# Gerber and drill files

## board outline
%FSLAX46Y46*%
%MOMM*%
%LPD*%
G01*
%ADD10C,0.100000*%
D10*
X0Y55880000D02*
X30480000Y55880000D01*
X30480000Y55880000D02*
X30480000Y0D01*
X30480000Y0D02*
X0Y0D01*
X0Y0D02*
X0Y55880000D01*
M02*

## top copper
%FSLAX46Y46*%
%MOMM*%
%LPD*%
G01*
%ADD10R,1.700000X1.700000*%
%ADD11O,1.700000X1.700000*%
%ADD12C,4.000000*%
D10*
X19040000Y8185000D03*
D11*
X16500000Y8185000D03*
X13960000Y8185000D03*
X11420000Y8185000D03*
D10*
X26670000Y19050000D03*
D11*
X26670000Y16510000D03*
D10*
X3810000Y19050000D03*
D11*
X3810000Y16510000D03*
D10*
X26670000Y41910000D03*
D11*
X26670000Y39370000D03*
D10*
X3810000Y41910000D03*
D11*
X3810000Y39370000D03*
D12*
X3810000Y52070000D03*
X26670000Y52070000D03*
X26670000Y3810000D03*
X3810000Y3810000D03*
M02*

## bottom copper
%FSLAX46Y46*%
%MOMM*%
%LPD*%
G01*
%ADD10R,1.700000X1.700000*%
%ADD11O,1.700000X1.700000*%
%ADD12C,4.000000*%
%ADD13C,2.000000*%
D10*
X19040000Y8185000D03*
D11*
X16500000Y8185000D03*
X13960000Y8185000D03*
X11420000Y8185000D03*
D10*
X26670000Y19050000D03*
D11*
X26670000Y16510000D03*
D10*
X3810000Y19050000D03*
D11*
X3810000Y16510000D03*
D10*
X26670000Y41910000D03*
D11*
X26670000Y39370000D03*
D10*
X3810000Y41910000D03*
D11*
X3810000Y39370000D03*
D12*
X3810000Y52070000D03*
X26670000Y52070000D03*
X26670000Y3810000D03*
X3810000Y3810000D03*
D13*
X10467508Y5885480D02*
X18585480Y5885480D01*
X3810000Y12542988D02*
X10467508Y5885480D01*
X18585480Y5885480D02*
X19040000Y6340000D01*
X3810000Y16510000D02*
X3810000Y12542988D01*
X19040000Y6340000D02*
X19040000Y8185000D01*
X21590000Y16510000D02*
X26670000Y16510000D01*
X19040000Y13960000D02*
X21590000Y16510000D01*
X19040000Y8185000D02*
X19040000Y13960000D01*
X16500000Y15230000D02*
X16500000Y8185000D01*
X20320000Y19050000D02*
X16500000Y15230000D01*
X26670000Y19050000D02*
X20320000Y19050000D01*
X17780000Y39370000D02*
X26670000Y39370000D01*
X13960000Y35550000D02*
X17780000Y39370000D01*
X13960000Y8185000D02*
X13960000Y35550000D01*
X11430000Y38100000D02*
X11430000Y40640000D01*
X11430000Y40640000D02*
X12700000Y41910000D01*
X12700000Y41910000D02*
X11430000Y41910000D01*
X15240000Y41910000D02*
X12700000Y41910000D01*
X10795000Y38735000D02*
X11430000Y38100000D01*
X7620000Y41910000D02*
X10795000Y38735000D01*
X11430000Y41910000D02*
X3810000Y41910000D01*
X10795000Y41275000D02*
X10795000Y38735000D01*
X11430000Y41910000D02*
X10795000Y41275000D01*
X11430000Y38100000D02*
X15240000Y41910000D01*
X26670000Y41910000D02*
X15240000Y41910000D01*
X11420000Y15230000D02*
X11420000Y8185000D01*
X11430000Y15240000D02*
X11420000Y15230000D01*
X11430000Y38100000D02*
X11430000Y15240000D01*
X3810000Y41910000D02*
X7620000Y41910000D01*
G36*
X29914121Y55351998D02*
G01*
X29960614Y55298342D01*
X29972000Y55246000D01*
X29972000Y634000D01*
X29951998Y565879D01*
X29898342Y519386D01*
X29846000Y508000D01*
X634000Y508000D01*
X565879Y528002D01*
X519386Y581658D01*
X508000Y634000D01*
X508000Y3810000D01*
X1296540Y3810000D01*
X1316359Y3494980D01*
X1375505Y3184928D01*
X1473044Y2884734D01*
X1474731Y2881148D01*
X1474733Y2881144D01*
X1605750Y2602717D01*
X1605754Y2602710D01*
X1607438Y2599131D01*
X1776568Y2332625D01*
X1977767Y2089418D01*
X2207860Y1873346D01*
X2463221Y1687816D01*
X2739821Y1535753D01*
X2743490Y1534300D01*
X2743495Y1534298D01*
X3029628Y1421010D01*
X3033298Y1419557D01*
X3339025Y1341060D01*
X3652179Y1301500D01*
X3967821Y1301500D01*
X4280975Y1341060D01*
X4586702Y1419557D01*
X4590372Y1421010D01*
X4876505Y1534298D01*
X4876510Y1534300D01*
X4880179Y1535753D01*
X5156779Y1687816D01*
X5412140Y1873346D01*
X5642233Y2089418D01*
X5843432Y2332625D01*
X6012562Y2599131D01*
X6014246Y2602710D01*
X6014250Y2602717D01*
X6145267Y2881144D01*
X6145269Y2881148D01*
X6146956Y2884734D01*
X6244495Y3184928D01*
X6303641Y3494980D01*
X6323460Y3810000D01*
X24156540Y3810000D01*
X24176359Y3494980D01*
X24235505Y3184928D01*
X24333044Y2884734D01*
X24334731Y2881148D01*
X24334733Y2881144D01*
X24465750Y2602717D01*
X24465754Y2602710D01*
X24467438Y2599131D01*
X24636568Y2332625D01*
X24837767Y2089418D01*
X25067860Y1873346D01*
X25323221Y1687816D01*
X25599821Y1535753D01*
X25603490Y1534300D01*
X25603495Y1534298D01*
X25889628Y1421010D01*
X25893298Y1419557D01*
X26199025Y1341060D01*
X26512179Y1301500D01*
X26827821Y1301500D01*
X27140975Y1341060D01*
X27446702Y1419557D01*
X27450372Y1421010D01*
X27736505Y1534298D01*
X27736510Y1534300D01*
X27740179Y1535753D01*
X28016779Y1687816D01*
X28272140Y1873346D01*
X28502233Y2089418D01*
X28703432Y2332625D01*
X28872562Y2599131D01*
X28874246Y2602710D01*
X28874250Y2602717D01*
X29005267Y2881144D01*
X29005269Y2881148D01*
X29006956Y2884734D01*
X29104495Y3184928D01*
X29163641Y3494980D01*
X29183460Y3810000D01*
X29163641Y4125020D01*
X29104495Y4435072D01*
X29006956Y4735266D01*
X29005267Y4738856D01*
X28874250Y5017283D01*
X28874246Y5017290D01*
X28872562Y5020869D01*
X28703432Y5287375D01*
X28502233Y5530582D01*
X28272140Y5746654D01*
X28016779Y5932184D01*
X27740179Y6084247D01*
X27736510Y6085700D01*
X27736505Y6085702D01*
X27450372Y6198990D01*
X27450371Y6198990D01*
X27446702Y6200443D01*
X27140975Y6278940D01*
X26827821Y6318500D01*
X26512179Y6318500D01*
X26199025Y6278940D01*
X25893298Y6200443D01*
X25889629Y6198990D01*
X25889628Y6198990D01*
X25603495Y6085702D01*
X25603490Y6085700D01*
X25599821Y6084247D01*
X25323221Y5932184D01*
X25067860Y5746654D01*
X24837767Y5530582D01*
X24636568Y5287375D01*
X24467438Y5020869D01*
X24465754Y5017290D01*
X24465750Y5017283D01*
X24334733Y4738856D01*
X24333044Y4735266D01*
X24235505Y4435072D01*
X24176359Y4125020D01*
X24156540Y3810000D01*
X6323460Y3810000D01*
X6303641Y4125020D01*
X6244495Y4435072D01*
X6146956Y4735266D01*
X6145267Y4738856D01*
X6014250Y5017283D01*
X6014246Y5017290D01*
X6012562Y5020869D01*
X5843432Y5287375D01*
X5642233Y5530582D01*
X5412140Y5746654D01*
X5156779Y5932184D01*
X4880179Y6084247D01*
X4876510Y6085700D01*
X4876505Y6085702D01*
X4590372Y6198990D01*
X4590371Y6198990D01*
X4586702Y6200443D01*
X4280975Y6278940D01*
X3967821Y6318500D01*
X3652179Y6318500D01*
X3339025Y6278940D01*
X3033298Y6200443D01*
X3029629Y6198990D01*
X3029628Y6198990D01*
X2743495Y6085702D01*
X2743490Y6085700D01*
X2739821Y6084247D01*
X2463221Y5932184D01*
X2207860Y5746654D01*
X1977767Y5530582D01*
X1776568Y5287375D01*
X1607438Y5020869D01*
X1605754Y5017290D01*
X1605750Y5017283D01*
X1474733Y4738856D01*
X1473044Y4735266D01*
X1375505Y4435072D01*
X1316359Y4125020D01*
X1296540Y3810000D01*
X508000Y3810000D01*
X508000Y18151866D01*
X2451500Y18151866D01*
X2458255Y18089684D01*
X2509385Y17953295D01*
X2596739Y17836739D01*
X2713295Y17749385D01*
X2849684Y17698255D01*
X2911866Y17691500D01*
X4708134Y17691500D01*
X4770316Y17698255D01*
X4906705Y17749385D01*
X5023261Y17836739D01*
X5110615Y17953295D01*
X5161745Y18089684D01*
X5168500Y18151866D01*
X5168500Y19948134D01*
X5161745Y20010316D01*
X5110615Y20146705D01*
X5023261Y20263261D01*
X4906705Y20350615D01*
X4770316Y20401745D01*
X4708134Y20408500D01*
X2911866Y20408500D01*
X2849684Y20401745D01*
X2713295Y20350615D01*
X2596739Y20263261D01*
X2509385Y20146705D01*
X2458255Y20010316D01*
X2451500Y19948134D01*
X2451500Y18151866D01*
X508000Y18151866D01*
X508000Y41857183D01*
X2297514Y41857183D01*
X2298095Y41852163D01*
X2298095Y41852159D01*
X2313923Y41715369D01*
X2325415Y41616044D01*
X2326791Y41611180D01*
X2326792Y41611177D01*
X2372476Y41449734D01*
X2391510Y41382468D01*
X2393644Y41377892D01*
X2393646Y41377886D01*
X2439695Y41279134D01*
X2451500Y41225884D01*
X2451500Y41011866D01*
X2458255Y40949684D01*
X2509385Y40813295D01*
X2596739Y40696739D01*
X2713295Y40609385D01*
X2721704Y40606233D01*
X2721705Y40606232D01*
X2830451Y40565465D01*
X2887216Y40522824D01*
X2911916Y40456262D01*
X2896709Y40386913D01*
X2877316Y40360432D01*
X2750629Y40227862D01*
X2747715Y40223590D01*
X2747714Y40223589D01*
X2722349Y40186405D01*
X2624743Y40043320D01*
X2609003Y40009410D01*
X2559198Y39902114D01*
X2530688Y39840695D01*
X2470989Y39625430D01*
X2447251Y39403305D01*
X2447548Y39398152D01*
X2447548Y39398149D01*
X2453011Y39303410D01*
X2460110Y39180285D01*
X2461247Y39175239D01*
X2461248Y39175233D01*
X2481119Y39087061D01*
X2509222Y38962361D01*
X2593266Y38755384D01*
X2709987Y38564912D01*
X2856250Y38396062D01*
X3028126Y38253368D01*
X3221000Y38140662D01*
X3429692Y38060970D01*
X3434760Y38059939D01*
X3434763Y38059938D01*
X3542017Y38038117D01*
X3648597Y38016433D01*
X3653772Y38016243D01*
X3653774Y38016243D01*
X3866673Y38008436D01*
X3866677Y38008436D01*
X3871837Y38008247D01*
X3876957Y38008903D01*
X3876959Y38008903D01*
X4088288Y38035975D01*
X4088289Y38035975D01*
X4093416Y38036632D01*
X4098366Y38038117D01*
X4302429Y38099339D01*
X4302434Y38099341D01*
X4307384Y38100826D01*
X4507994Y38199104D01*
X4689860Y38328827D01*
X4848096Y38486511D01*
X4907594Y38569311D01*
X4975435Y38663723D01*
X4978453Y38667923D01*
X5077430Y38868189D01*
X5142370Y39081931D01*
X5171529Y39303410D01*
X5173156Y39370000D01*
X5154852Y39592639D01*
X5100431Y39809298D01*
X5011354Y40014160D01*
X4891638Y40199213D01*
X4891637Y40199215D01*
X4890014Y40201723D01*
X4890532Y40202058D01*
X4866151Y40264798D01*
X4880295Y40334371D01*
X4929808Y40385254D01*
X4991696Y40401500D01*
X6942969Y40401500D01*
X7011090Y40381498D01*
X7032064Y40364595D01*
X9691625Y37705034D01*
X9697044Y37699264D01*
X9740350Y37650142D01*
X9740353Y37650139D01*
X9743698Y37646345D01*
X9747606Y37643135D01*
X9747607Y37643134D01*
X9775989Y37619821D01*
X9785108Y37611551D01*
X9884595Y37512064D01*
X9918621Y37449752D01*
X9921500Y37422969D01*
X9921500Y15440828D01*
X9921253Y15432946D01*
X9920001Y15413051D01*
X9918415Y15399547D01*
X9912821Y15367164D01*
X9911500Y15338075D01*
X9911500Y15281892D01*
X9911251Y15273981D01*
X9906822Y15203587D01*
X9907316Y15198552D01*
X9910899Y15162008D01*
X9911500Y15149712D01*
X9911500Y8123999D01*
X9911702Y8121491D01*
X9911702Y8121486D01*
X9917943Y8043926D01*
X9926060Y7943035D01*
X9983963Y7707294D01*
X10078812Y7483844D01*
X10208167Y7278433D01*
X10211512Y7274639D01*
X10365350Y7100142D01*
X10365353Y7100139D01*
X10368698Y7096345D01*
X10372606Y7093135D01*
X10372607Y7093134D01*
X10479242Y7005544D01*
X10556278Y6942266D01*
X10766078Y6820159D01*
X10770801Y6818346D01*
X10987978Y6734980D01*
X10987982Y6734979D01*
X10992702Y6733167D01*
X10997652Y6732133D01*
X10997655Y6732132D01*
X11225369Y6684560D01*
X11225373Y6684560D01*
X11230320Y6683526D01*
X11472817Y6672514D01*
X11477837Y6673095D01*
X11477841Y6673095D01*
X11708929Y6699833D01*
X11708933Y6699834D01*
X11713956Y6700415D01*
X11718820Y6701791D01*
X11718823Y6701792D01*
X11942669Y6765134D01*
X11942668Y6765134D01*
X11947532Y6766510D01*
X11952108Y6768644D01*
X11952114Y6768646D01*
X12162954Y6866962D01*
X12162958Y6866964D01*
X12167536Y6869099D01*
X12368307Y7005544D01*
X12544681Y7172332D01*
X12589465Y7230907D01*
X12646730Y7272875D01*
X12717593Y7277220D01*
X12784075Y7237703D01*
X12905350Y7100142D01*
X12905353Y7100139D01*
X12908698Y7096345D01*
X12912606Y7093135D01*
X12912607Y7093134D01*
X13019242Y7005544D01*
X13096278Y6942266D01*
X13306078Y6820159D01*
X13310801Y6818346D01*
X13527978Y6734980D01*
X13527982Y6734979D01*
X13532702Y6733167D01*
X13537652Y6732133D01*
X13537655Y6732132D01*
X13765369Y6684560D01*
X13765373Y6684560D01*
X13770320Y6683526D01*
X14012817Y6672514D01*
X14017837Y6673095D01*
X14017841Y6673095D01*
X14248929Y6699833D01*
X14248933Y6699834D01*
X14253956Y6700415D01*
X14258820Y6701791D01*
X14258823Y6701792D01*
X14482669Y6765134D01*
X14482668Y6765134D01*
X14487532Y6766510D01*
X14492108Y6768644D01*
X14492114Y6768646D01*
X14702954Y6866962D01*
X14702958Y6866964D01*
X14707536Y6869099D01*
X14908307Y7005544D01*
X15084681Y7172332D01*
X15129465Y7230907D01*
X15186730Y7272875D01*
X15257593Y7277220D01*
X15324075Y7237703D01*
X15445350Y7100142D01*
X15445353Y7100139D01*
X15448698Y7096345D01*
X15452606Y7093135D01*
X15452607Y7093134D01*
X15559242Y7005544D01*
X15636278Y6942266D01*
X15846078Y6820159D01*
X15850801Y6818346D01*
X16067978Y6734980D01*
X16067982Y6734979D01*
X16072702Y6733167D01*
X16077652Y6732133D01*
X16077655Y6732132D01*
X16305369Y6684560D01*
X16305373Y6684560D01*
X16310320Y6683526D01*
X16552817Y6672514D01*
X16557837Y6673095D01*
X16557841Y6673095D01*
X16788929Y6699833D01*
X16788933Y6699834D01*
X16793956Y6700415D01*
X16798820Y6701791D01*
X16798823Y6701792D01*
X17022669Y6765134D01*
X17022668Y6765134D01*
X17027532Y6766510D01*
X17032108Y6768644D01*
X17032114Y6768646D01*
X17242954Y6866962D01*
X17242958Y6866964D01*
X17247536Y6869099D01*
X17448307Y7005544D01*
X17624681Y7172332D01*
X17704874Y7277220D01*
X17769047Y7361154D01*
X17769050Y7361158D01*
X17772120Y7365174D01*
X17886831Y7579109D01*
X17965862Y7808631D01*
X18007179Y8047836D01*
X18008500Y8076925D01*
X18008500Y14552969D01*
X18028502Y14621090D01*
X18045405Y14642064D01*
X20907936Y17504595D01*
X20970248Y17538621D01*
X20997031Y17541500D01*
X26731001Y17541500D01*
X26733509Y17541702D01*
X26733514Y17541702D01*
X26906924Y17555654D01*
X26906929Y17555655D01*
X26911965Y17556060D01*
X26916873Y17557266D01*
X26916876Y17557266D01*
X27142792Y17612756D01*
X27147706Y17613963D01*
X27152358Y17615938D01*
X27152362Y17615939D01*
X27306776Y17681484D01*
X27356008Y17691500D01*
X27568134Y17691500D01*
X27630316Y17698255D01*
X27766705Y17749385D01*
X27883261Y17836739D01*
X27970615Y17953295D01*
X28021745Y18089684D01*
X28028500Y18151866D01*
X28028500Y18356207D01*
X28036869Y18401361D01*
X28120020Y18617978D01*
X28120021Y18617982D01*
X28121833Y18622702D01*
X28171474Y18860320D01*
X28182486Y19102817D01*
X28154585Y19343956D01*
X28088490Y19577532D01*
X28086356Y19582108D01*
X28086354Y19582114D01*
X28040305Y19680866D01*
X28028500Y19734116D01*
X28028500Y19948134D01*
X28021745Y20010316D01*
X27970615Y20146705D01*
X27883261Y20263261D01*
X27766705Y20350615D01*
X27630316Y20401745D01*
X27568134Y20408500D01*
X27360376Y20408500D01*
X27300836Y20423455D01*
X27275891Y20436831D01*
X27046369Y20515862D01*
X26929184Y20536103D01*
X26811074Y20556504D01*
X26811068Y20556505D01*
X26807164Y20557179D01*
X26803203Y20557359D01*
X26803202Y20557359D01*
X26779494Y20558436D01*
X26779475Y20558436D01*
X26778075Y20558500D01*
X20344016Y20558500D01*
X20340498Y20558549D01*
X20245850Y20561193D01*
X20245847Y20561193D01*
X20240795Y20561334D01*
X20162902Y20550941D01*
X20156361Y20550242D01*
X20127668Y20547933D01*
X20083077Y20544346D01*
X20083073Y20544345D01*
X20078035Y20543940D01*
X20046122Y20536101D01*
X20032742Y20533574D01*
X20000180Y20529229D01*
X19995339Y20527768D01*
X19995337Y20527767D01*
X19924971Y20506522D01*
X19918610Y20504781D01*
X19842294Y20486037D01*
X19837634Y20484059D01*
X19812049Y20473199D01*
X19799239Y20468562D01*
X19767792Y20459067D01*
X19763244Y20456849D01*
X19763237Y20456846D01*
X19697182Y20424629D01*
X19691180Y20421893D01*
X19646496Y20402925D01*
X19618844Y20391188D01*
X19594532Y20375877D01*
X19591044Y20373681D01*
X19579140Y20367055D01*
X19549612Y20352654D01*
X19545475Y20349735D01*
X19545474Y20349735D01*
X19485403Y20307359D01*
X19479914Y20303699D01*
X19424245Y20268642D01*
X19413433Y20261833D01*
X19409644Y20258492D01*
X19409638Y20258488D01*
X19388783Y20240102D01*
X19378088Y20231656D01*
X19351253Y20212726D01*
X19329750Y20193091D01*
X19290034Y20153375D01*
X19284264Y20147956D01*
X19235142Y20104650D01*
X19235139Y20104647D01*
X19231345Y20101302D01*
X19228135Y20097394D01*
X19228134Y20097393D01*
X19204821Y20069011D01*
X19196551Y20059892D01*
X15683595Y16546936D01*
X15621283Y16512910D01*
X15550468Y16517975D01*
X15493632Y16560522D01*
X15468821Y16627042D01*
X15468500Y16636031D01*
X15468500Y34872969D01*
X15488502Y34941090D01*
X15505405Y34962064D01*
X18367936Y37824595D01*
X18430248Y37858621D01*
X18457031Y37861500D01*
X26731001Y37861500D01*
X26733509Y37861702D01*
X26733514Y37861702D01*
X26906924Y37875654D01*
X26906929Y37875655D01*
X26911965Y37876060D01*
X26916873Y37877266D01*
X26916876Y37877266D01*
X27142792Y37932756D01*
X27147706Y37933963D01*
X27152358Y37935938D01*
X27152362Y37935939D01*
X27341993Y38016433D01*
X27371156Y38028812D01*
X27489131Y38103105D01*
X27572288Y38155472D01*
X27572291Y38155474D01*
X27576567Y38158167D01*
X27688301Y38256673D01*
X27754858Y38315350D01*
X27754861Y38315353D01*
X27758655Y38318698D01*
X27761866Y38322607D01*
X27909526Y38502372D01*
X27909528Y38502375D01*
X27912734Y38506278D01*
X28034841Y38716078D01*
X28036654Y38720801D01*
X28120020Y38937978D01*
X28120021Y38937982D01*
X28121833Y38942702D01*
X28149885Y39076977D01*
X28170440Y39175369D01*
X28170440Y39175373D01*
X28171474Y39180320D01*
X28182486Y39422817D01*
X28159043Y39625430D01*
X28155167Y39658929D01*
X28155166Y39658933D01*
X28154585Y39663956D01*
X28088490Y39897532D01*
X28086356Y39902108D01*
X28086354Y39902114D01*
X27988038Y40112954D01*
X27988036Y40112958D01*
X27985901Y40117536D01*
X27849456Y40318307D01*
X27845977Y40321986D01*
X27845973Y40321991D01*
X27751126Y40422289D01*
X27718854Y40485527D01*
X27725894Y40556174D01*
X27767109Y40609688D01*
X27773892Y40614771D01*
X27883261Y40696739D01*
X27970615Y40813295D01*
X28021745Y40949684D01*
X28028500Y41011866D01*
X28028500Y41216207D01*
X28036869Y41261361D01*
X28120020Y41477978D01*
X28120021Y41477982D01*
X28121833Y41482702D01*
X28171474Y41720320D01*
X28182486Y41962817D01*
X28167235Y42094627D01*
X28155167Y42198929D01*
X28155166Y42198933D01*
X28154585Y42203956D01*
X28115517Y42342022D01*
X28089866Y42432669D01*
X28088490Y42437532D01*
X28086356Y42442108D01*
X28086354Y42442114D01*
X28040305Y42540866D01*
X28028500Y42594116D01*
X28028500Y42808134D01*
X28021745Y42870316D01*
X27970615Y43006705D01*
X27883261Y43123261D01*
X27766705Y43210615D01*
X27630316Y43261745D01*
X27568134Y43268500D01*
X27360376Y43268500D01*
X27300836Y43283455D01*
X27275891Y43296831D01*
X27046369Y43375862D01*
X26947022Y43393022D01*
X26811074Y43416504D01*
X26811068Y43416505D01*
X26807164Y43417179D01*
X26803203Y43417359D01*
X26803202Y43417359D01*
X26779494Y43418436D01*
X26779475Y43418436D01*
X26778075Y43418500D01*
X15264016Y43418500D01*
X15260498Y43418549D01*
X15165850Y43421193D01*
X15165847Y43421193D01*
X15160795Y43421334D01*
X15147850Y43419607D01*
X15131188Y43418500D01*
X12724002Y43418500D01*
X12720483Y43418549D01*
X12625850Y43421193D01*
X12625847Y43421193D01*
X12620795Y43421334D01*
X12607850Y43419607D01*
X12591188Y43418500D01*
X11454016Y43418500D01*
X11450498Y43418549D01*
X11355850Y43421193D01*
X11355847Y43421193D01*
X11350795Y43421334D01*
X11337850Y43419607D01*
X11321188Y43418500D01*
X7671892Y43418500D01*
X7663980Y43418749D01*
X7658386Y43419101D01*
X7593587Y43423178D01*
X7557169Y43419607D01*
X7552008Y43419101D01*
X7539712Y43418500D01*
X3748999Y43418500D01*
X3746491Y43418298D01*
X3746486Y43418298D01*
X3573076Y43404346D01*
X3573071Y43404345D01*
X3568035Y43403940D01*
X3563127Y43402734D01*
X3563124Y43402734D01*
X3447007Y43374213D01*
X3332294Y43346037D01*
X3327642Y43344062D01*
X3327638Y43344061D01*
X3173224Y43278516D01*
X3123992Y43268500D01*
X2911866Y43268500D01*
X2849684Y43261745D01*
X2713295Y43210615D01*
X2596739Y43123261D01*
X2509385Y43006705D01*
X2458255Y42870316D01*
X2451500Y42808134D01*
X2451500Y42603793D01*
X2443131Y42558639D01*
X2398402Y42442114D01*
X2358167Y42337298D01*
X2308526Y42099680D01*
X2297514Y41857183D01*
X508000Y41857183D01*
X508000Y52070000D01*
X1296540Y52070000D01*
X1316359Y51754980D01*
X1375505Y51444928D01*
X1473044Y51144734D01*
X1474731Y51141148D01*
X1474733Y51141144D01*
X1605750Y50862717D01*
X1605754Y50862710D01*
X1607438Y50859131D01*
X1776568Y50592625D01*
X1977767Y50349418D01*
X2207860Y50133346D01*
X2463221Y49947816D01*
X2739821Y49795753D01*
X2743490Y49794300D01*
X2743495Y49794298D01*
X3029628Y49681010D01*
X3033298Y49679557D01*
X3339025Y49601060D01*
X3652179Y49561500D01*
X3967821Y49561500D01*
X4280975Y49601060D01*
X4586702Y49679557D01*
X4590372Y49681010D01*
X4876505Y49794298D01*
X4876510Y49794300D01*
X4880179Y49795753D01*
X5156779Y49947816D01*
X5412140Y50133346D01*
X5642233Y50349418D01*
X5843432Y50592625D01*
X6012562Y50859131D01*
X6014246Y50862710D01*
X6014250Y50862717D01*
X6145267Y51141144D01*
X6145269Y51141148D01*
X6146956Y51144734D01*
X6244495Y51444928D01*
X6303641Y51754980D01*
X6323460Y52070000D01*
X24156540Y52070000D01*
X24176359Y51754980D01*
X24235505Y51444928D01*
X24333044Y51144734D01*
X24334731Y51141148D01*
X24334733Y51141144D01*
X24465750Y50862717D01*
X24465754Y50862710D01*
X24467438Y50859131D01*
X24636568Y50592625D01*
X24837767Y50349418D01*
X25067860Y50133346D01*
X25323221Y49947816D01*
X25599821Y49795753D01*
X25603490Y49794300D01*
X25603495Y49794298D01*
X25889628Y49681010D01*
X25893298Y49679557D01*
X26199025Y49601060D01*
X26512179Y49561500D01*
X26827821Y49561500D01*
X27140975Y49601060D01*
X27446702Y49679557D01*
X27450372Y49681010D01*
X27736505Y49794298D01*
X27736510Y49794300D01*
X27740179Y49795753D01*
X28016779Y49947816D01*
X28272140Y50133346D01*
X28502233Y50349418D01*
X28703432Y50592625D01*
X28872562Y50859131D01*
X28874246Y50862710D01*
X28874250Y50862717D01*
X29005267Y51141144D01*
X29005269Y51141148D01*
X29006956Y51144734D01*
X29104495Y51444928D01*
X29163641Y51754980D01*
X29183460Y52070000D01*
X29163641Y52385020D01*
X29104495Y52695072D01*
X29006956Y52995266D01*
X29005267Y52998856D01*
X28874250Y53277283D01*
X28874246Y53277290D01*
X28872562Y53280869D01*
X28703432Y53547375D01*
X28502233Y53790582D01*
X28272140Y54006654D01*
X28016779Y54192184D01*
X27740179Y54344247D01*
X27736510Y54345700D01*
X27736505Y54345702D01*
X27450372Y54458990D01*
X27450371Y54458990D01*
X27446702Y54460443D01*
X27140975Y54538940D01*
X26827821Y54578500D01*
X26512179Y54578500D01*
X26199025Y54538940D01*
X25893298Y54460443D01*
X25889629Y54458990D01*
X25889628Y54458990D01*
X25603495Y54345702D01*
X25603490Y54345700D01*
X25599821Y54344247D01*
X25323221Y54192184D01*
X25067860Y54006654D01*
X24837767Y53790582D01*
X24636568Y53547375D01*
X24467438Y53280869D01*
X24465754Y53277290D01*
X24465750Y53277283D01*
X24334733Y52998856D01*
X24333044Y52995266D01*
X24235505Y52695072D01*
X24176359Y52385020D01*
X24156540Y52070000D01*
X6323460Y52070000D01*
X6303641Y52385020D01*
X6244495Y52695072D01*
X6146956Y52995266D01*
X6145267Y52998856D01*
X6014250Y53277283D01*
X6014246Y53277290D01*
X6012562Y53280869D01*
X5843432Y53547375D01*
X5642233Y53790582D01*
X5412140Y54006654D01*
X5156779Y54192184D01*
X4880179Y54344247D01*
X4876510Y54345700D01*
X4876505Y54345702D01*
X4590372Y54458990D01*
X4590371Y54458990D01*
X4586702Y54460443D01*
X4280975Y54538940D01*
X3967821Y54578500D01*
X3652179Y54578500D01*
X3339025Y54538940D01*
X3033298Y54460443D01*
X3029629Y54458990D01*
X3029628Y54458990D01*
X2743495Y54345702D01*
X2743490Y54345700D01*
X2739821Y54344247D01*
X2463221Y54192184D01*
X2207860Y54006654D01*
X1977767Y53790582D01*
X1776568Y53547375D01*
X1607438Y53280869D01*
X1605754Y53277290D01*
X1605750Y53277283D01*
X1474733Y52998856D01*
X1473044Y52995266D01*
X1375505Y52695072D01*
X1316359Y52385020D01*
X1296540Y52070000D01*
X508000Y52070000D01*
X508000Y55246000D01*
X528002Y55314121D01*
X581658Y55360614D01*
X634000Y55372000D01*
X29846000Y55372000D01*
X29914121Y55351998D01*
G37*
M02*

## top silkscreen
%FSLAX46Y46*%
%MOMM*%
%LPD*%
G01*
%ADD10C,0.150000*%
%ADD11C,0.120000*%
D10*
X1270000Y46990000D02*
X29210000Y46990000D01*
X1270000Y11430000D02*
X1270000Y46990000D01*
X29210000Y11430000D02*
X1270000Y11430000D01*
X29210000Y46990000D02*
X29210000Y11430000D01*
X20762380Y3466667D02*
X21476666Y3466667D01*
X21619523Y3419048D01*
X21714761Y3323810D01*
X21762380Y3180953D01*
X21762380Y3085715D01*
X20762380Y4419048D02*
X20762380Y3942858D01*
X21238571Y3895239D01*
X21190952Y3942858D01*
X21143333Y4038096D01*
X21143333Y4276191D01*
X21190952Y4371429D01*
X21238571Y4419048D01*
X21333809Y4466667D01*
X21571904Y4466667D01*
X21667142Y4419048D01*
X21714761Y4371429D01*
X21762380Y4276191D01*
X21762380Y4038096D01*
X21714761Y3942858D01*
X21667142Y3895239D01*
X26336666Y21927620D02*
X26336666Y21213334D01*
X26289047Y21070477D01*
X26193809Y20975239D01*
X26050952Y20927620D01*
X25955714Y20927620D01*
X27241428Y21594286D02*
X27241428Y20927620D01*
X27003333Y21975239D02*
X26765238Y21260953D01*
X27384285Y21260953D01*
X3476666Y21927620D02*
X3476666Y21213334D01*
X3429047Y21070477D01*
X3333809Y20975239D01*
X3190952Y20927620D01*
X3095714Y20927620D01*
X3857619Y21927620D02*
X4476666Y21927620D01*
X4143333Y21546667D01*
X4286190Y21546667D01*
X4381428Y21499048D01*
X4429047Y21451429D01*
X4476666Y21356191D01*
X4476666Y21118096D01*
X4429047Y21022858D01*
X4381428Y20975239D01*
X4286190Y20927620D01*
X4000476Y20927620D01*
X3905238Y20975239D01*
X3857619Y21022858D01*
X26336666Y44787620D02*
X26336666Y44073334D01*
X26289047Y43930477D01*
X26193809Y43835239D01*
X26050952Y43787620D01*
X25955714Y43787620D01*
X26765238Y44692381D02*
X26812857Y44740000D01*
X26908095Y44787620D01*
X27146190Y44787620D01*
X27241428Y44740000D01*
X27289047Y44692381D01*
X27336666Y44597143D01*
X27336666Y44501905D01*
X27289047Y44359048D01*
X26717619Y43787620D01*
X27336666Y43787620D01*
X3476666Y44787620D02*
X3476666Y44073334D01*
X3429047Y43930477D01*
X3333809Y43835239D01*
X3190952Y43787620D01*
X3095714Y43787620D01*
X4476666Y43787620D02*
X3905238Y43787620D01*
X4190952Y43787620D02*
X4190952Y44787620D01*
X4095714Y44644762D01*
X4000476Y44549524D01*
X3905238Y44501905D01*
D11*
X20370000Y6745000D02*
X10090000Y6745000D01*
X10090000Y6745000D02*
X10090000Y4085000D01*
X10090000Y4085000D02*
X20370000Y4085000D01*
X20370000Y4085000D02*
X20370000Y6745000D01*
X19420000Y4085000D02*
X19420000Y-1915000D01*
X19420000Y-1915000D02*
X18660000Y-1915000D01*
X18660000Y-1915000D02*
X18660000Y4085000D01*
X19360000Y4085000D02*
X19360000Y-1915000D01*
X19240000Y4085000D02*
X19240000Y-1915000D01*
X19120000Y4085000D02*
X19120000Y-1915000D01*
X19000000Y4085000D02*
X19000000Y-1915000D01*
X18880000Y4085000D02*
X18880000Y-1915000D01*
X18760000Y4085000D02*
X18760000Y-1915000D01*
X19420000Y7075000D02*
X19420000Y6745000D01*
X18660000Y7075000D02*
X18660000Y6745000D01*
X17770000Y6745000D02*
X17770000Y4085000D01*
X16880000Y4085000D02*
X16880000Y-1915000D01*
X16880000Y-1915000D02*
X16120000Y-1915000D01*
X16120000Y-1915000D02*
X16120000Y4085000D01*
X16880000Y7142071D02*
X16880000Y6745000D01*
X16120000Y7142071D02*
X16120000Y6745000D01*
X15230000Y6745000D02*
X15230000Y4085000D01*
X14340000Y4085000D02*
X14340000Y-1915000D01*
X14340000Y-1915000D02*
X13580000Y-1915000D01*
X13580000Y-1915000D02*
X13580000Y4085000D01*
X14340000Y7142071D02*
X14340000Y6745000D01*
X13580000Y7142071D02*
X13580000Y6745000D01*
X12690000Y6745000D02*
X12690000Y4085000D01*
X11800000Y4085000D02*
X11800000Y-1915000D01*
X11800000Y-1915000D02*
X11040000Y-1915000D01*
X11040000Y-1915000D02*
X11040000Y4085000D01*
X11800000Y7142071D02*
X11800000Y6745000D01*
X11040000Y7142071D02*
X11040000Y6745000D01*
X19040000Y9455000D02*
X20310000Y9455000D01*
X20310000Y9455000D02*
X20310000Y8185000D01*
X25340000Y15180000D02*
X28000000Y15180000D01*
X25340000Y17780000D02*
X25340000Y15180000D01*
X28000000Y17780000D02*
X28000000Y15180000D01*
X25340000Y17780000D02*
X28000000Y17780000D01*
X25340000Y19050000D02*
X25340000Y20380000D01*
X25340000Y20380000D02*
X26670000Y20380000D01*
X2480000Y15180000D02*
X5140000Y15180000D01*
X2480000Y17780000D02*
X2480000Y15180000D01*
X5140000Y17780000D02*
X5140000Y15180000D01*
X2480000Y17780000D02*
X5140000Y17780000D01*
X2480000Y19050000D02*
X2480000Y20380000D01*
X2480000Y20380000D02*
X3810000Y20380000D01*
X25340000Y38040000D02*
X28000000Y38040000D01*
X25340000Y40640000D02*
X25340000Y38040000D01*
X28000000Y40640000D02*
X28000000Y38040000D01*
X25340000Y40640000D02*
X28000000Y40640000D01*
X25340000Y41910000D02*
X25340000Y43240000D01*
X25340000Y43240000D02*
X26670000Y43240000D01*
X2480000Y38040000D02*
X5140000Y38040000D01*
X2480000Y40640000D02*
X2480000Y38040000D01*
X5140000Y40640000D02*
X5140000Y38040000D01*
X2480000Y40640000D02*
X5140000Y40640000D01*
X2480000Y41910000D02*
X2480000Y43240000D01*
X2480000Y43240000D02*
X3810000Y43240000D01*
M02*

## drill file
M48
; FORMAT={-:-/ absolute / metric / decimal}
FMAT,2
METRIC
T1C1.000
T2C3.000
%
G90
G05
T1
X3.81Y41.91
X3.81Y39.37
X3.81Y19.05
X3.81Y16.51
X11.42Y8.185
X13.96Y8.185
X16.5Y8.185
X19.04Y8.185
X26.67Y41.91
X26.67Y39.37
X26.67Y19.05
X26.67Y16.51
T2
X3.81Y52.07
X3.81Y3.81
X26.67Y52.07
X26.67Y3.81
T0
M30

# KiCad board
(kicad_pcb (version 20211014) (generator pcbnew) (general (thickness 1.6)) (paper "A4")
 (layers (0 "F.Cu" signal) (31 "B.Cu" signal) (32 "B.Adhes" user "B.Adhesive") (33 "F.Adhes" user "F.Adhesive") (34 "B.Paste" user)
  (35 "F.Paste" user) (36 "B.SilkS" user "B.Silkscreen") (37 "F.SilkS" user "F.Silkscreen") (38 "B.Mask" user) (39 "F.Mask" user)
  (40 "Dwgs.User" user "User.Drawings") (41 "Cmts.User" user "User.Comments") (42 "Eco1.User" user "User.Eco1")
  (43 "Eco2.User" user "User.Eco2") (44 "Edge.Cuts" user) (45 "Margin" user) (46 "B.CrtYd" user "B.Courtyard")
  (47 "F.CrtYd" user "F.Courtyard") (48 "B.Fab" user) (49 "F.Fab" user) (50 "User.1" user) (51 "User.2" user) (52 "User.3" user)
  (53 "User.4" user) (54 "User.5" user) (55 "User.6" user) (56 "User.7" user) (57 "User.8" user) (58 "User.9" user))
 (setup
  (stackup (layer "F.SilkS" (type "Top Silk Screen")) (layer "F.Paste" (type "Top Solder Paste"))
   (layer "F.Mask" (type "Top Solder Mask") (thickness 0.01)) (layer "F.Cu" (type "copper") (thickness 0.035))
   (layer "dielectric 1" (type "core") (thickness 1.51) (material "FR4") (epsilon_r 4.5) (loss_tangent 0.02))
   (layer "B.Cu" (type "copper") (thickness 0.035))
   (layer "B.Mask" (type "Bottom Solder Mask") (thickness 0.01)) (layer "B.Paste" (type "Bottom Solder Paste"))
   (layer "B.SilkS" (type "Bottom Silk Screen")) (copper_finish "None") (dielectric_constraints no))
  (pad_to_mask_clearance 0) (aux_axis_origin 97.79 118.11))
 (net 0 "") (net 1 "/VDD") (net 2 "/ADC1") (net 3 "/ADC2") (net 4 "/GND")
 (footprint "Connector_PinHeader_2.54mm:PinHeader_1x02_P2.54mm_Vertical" (layer "F.Cu") (at 101.6 76.2)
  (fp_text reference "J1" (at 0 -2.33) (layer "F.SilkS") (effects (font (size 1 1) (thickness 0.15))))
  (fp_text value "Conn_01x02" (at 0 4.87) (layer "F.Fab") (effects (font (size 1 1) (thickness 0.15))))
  (fp_line (start -1.33 3.87) (end 1.33 3.87) (layer "F.SilkS") (width 0.12))
  (fp_line (start -1.33 1.27) (end -1.33 3.87) (layer "F.SilkS") (width 0.12))
  (fp_line (start 1.33 1.27) (end 1.33 3.87) (layer "F.SilkS") (width 0.12))
  (fp_line (start -1.33 1.27) (end 1.33 1.27) (layer "F.SilkS") (width 0.12))
  (fp_line (start -1.33 0) (end -1.33 -1.33) (layer "F.SilkS") (width 0.12))
  (fp_line (start -1.33 -1.33) (end 0 -1.33) (layer "F.SilkS") (width 0.12))
  (pad "1" thru_hole rect locked (at 0 0) (size 1.7 1.7) (drill 1) (layers *.Cu *.Mask) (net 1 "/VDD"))
  (pad "2" thru_hole oval locked (at 0 2.54) (size 1.7 1.7) (drill 1) (layers *.Cu *.Mask) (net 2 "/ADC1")))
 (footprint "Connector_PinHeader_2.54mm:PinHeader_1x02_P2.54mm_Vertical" (layer "F.Cu") (at 124.46 99.06)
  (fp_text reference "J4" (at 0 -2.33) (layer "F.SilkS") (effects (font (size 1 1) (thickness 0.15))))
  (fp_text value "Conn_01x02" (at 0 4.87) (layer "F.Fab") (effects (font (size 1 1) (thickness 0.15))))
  (fp_line (start -1.33 -1.33) (end 0 -1.33) (layer "F.SilkS") (width 0.12))
  (fp_line (start 1.33 1.27) (end 1.33 3.87) (layer "F.SilkS") (width 0.12))
  (fp_line (start -1.33 1.27) (end -1.33 3.87) (layer "F.SilkS") (width 0.12))
  (fp_line (start -1.33 3.87) (end 1.33 3.87) (layer "F.SilkS") (width 0.12))
  (fp_line (start -1.33 0) (end -1.33 -1.33) (layer "F.SilkS") (width 0.12))
  (fp_line (start -1.33 1.27) (end 1.33 1.27) (layer "F.SilkS") (width 0.12))
  (pad "1" thru_hole rect locked (at 0 0) (size 1.7 1.7) (drill 1) (layers *.Cu *.Mask) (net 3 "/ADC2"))
  (pad "2" thru_hole oval locked (at 0 2.54) (size 1.7 1.7) (drill 1) (layers *.Cu *.Mask) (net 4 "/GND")))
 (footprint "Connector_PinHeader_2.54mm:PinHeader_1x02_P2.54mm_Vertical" (layer "F.Cu") (at 124.46 76.2)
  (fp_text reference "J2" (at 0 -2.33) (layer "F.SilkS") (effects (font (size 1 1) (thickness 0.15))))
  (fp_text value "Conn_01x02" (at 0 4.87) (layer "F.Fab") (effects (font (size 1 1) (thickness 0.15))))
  (fp_line (start -1.33 -1.33) (end 0 -1.33) (layer "F.SilkS") (width 0.12))
  (fp_line (start -1.33 0) (end -1.33 -1.33) (layer "F.SilkS") (width 0.12))
  (fp_line (start -1.33 1.27) (end -1.33 3.87) (layer "F.SilkS") (width 0.12))
  (fp_line (start -1.33 3.87) (end 1.33 3.87) (layer "F.SilkS") (width 0.12))
  (fp_line (start -1.33 1.27) (end 1.33 1.27) (layer "F.SilkS") (width 0.12))
  (fp_line (start 1.33 1.27) (end 1.33 3.87) (layer "F.SilkS") (width 0.12))
  (pad "1" thru_hole rect locked (at 0 0) (size 1.7 1.7) (drill 1) (layers *.Cu *.Mask) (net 1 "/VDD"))
  (pad "2" thru_hole oval locked (at 0 2.54) (size 1.7 1.7) (drill 1) (layers *.Cu *.Mask) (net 2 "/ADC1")))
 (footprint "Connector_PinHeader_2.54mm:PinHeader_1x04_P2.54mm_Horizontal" (layer "F.Cu") (at 116.83 109.925 -90)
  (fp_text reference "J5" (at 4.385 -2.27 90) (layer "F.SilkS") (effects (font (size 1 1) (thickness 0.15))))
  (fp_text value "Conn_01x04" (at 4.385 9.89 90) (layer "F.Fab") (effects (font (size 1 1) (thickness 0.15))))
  (fp_line (start 10.1 5.46) (end 4.1 5.46) (layer "F.SilkS") (width 0.12))
  (fp_line (start 10.1 0.38) (end 4.1 0.38) (layer "F.SilkS") (width 0.12))
  (fp_line (start 1.11 0.38) (end 1.44 0.38) (layer "F.SilkS") (width 0.12))
  (fp_line (start 10.1 2.92) (end 4.1 2.92) (layer "F.SilkS") (width 0.12))
  (fp_line (start 10.1 4.7) (end 10.1 5.46) (layer "F.SilkS") (width 0.12))
  (fp_line (start 1.042929 2.16) (end 1.44 2.16) (layer "F.SilkS") (width 0.12))
  (fp_line (start 1.042929 5.46) (end 1.44 5.46) (layer "F.SilkS") (width 0.12))
  (fp_line (start 1.44 3.81) (end 4.1 3.81) (layer "F.SilkS") (width 0.12))
  (fp_line (start 10.1 8) (end 4.1 8) (layer "F.SilkS") (width 0.12))
  (fp_line (start 4.1 0.04) (end 10.1 0.04) (layer "F.SilkS") (width 0.12))
  (fp_line (start 4.1 -0.32) (end 10.1 -0.32) (layer "F.SilkS") (width 0.12))
  (fp_line (start 4.1 0.16) (end 10.1 0.16) (layer "F.SilkS") (width 0.12))
  (fp_line (start 1.042929 4.7) (end 1.44 4.7) (layer "F.SilkS") (width 0.12))
  (fp_line (start 1.44 8.95) (end 4.1 8.95) (layer "F.SilkS") (width 0.12))
  (fp_line (start 1.042929 2.92) (end 1.44 2.92) (layer "F.SilkS") (width 0.12))
  (fp_line (start 10.1 2.16) (end 10.1 2.92) (layer "F.SilkS") (width 0.12))
  (fp_line (start 4.1 -0.2) (end 10.1 -0.2) (layer "F.SilkS") (width 0.12))
  (fp_line (start 10.1 7.24) (end 10.1 8) (layer "F.SilkS") (width 0.12))
  (fp_line (start 1.44 -1.33) (end 1.44 8.95) (layer "F.SilkS") (width 0.12))
  (fp_line (start 1.44 6.35) (end 4.1 6.35) (layer "F.SilkS") (width 0.12))
  (fp_line (start 4.1 -0.08) (end 10.1 -0.08) (layer "F.SilkS") (width 0.12))
  (fp_line (start -1.27 -1.27) (end 0 -1.27) (layer "F.SilkS") (width 0.12))
  (fp_line (start 1.11 -0.38) (end 1.44 -0.38) (layer "F.SilkS") (width 0.12))
  (fp_line (start -1.27 0) (end -1.27 -1.27) (layer "F.SilkS") (width 0.12))
  (fp_line (start 4.1 0.28) (end 10.1 0.28) (layer "F.SilkS") (width 0.12))
  (fp_line (start 1.042929 8) (end 1.44 8) (layer "F.SilkS") (width 0.12))
  (fp_line (start 1.042929 7.24) (end 1.44 7.24) (layer "F.SilkS") (width 0.12))
  (fp_line (start 4.1 2.16) (end 10.1 2.16) (layer "F.SilkS") (width 0.12))
  (fp_line (start 4.1 8.95) (end 4.1 -1.33) (layer "F.SilkS") (width 0.12))
  (fp_line (start 4.1 -0.38) (end 10.1 -0.38) (layer "F.SilkS") (width 0.12))
  (fp_line (start 1.44 1.27) (end 4.1 1.27) (layer "F.SilkS") (width 0.12))
  (fp_line (start 4.1 4.7) (end 10.1 4.7) (layer "F.SilkS") (width 0.12))
  (fp_line (start 4.1 7.24) (end 10.1 7.24) (layer "F.SilkS") (width 0.12))
  (fp_line (start 10.1 -0.38) (end 10.1 0.38) (layer "F.SilkS") (width 0.12))
  (fp_line (start 4.1 -1.33) (end 1.44 -1.33) (layer "F.SilkS") (width 0.12))
  (pad "1" thru_hole rect locked (at 0 0 270) (size 1.7 1.7) (drill 1) (layers *.Cu *.Mask) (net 4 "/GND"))
  (pad "2" thru_hole oval locked (at 0 2.54 270) (size 1.7 1.7) (drill 1) (layers *.Cu *.Mask) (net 3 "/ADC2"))
  (pad "3" thru_hole oval locked (at 0 5.08 270) (size 1.7 1.7) (drill 1) (layers *.Cu *.Mask) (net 2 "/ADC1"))
  (pad "4" thru_hole oval locked (at 0 7.62 270) (size 1.7 1.7) (drill 1) (layers *.Cu *.Mask) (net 1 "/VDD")))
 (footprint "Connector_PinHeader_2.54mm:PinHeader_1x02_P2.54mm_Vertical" (layer "F.Cu") (at 101.6 99.06)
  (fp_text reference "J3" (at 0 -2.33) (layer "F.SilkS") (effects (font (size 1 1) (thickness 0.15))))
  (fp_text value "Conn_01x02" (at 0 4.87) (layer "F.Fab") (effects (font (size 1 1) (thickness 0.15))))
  (fp_line (start -1.33 3.87) (end 1.33 3.87) (layer "F.SilkS") (width 0.12))
  (fp_line (start -1.33 1.27) (end -1.33 3.87) (layer "F.SilkS") (width 0.12))
  (fp_line (start -1.33 -1.33) (end 0 -1.33) (layer "F.SilkS") (width 0.12))
  (fp_line (start -1.33 0) (end -1.33 -1.33) (layer "F.SilkS") (width 0.12))
  (fp_line (start -1.33 1.27) (end 1.33 1.27) (layer "F.SilkS") (width 0.12))
  (fp_line (start 1.33 1.27) (end 1.33 3.87) (layer "F.SilkS") (width 0.12))
  (pad "1" thru_hole rect locked (at 0 0) (size 1.7 1.7) (drill 1) (layers *.Cu *.Mask) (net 3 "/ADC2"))
  (pad "2" thru_hole oval locked (at 0 2.54) (size 1.7 1.7) (drill 1) (layers *.Cu *.Mask) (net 4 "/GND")))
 (gr_line (start 127 71.12) (end 127 106.68) (layer "F.SilkS") (width 0.15))
 (gr_line (start 127 106.68) (end 99.06 106.68) (layer "F.SilkS") (width 0.15))
 (gr_line (start 99.06 71.12) (end 127 71.12) (layer "F.SilkS") (width 0.15))
 (gr_line (start 99.06 106.68) (end 99.06 71.12) (layer "F.SilkS") (width 0.15))
 (gr_rect (start 97.79 62.23) (end 128.27 118.11) (layer "Edge.Cuts") (width 0.1) (fill none))
 (via (at 124.46 66.04) (size 4) (drill 3) (layers "F.Cu" "B.Cu") (free) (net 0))
 (via (at 124.46 114.3) (size 4) (drill 3) (layers "F.Cu" "B.Cu") (free) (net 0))
 (via (at 101.6 114.3) (size 4) (drill 3) (layers "F.Cu" "B.Cu") (free) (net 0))
 (via (at 101.6 66.04) (size 4) (drill 3) (layers "F.Cu" "B.Cu") (free) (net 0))
 (segment (start 109.22 76.2) (end 108.585 76.835) (width 2) (layer "B.Cu") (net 1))
 (segment (start 109.22 102.87) (end 109.21 102.88) (width 2) (layer "B.Cu") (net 1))
 (segment (start 110.49 76.2) (end 109.22 76.2) (width 2) (layer "B.Cu") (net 1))
 (segment (start 101.6 76.2) (end 105.41 76.2) (width 2) (layer "B.Cu") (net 1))
 (segment (start 108.585 79.375) (end 109.22 80.01) (width 2) (layer "B.Cu") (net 1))
 (segment (start 109.22 80.01) (end 113.03 76.2) (width 2) (layer "B.Cu") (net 1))
 (segment (start 109.22 80.01) (end 109.22 77.47) (width 2) (layer "B.Cu") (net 1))
 (segment (start 109.21 102.88) (end 109.21 109.925) (width 2) (layer "B.Cu") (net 1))
 (segment (start 109.22 76.2) (end 101.6 76.2) (width 2) (layer "B.Cu") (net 1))
 (segment (start 108.585 76.835) (end 108.585 79.375) (width 2) (layer "B.Cu") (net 1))
 (segment (start 105.41 76.2) (end 108.585 79.375) (width 2) (layer "B.Cu") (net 1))
 (segment (start 109.22 80.01) (end 109.22 102.87) (width 2) (layer "B.Cu") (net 1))
 (segment (start 109.22 77.47) (end 110.49 76.2) (width 2) (layer "B.Cu") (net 1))
 (segment (start 124.46 76.2) (end 113.03 76.2) (width 2) (layer "B.Cu") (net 1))
 (segment (start 113.03 76.2) (end 110.49 76.2) (width 2) (layer "B.Cu") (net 1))
 (segment (start 111.75 82.56) (end 115.57 78.74) (width 2) (layer "B.Cu") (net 2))
 (segment (start 111.75 109.925) (end 111.75 82.56) (width 2) (layer "B.Cu") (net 2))
 (segment (start 115.57 78.74) (end 124.46 78.74) (width 2) (layer "B.Cu") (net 2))
 (segment (start 118.11 99.06) (end 114.29 102.88) (width 2) (layer "B.Cu") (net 3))
 (segment (start 124.46 99.06) (end 118.11 99.06) (width 2) (layer "B.Cu") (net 3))
 (segment (start 114.29 102.88) (end 114.29 109.925) (width 2) (layer "B.Cu") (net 3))
 (segment (start 116.83 111.77) (end 116.83 109.925) (width 2) (layer "B.Cu") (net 4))
 (segment (start 116.83 104.15) (end 119.38 101.6) (width 2) (layer "B.Cu") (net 4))
 (segment (start 119.38 101.6) (end 124.46 101.6) (width 2) (layer "B.Cu") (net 4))
 (segment (start 101.6 101.6) (end 101.6 105.567012) (width 2) (layer "B.Cu") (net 4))
 (segment (start 116.83 109.925) (end 116.83 104.15) (width 2) (layer "B.Cu") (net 4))
 (segment (start 101.6 105.567012) (end 108.257508 112.22452) (width 2) (layer "B.Cu") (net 4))
 (segment (start 116.37548 112.22452) (end 116.83 111.77) (width 2) (layer "B.Cu") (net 4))
 (segment (start 108.257508 112.22452) (end 116.37548 112.22452) (width 2) (layer "B.Cu") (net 4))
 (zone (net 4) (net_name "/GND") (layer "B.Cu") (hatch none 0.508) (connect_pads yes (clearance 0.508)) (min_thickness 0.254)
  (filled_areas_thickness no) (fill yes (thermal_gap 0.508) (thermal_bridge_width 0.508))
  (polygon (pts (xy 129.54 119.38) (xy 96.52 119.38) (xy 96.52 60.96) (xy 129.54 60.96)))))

